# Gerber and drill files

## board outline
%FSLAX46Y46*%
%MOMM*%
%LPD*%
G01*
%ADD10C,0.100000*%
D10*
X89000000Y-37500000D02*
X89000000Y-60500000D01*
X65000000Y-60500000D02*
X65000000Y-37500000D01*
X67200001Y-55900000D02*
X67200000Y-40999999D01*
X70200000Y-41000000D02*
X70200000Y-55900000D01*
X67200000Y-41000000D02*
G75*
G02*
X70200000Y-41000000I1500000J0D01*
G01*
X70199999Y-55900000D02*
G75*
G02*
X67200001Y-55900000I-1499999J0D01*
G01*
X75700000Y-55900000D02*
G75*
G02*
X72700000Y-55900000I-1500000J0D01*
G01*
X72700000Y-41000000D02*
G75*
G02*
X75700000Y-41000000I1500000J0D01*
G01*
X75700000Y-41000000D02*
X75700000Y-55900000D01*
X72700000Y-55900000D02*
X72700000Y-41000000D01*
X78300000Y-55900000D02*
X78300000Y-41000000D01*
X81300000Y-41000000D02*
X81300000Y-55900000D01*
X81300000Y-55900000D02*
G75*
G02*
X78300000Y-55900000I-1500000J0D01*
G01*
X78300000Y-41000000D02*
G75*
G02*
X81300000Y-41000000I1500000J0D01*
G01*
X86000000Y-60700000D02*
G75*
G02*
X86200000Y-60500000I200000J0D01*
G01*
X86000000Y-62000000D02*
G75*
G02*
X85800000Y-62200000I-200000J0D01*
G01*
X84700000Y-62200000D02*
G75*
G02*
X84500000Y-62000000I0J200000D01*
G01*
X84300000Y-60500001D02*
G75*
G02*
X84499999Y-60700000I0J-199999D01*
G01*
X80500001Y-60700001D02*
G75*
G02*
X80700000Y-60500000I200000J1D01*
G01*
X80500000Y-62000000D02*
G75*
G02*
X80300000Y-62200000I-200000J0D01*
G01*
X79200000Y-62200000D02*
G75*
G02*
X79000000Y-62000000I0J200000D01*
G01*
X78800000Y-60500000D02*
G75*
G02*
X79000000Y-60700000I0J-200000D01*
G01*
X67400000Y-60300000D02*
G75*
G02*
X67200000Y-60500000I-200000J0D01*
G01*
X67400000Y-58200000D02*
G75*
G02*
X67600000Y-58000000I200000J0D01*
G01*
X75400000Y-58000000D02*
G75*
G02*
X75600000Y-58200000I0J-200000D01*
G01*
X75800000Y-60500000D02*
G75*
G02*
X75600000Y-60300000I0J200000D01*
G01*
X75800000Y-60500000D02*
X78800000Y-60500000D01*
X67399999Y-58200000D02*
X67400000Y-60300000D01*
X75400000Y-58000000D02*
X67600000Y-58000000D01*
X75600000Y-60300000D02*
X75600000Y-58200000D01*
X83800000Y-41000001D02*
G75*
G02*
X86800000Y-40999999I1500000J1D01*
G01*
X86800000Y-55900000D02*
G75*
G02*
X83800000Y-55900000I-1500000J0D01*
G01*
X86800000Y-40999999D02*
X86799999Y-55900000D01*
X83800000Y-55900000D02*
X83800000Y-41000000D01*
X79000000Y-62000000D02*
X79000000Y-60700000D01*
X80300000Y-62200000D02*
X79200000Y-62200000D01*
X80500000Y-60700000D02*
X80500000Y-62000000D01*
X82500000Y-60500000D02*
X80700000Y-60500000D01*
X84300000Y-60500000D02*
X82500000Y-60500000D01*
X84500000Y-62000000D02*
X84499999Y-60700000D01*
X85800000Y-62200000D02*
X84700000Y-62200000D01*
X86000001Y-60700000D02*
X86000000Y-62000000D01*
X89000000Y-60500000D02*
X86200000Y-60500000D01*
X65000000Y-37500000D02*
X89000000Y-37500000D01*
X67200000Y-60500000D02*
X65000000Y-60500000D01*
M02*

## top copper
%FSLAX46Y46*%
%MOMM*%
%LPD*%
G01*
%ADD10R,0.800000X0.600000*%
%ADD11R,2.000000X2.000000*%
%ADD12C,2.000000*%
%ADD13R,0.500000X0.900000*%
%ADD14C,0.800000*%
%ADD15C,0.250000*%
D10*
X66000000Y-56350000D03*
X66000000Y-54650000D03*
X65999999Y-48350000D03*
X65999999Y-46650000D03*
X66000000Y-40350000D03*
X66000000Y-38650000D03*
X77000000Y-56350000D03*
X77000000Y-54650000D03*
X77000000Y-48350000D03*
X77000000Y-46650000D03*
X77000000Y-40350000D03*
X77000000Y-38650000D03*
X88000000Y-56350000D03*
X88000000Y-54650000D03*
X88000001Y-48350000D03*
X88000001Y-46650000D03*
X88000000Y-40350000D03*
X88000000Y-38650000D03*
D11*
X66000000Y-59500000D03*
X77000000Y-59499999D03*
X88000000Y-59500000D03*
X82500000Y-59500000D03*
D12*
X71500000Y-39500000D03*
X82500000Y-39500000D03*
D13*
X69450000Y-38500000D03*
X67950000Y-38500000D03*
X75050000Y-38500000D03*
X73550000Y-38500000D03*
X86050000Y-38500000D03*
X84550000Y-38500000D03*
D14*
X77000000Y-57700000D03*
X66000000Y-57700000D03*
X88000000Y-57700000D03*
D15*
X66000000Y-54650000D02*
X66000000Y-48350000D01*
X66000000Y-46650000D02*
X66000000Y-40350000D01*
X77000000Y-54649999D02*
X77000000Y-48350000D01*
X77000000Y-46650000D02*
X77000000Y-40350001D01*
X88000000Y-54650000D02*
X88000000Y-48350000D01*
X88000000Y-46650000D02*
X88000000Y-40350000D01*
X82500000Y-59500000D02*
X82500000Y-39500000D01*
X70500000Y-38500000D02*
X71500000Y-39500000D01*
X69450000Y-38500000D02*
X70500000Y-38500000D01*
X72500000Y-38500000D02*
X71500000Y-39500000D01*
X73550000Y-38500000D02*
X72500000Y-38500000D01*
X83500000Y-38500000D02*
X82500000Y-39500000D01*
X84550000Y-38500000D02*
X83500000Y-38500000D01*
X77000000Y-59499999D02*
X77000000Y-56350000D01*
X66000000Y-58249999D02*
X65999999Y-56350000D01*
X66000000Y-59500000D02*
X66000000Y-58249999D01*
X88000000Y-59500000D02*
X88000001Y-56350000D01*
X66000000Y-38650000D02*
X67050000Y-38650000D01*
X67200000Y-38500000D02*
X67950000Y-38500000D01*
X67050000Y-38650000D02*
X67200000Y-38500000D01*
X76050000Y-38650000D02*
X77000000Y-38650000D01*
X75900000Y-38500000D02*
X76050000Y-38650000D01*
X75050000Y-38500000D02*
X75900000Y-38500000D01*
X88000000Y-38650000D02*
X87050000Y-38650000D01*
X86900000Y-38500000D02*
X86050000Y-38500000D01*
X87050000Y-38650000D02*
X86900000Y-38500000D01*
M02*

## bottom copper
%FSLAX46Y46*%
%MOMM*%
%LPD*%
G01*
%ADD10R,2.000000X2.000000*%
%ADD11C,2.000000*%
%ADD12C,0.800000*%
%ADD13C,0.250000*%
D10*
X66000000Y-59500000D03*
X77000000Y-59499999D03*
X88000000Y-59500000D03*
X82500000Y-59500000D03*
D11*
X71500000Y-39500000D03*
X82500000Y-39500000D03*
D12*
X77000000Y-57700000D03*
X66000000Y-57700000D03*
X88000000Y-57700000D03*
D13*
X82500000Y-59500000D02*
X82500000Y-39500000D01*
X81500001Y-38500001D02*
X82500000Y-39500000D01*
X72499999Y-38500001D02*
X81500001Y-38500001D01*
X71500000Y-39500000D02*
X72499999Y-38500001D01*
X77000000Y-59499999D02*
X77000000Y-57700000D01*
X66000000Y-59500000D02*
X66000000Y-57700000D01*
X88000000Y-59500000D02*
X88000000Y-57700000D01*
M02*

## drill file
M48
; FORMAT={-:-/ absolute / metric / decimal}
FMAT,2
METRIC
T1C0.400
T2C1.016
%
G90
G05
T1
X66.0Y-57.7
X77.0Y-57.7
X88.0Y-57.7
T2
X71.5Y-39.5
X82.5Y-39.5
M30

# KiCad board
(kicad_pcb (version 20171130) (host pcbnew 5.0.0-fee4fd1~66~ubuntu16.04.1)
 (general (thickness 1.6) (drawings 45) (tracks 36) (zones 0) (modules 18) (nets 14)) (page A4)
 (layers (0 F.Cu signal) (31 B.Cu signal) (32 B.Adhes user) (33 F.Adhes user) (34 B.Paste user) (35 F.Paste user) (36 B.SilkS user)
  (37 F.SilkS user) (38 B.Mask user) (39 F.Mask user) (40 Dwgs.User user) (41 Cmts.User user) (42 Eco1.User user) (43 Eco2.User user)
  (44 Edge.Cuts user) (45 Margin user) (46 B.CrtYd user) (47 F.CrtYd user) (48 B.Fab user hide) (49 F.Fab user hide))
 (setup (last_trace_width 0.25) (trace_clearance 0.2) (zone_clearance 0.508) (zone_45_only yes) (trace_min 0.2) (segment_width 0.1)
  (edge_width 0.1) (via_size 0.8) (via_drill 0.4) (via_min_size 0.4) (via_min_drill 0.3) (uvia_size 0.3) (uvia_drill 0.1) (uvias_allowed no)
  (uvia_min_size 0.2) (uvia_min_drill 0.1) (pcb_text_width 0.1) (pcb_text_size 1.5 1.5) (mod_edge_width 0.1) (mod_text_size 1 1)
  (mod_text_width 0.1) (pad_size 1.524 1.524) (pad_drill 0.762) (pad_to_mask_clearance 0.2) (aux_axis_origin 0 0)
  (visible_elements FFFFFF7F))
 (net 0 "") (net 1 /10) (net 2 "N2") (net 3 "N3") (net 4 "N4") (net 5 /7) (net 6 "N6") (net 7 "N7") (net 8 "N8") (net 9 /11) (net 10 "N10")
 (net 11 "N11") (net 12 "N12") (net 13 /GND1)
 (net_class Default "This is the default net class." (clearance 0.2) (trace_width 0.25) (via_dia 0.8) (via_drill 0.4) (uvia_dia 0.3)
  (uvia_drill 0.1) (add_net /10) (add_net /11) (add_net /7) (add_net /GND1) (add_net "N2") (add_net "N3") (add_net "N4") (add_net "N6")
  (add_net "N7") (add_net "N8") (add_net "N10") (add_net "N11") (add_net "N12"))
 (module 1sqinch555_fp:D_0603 (layer F.Cu) (at 66 55.5 270)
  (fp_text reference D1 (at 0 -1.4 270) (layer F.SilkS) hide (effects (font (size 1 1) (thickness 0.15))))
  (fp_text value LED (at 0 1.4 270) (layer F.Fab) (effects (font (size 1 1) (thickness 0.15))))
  (pad 2 smd rect (at 0.85 0 270) (size 0.6 0.8) (layers F.Cu F.Paste F.Mask) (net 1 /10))
  (pad 1 smd rect (at -0.85 0 270) (size 0.6 0.8) (layers F.Cu F.Paste F.Mask) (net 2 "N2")))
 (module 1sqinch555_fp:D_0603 (layer F.Cu) (at 65.999999 47.5 270)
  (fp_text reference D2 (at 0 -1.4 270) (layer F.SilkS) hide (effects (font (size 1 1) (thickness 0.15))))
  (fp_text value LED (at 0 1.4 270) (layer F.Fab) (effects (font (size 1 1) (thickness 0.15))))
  (pad 2 smd rect (at 0.85 0 270) (size 0.6 0.8) (layers F.Cu F.Paste F.Mask) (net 2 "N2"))
  (pad 1 smd rect (at -0.85 0 270) (size 0.6 0.8) (layers F.Cu F.Paste F.Mask) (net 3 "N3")))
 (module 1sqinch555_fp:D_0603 (layer F.Cu) (at 66 39.5 270)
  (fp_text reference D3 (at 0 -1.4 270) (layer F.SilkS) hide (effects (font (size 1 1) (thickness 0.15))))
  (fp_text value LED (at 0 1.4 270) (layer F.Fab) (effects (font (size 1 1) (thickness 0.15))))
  (pad 2 smd rect (at 0.85 0 270) (size 0.6 0.8) (layers F.Cu F.Paste F.Mask) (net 3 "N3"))
  (pad 1 smd rect (at -0.85 0 270) (size 0.6 0.8) (layers F.Cu F.Paste F.Mask) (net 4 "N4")))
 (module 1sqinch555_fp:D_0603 (layer F.Cu) (at 77 55.5 270)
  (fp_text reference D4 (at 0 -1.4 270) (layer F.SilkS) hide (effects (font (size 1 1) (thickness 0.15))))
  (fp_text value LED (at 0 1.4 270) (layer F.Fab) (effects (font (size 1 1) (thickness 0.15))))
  (pad 2 smd rect (at 0.85 0 270) (size 0.6 0.8) (layers F.Cu F.Paste F.Mask) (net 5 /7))
  (pad 1 smd rect (at -0.85 0 270) (size 0.6 0.8) (layers F.Cu F.Paste F.Mask) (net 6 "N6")))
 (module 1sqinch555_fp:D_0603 (layer F.Cu) (at 77 47.5 270)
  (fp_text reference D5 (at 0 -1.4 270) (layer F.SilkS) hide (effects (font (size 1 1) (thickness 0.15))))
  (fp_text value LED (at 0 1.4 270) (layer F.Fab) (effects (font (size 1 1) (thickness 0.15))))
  (pad 2 smd rect (at 0.85 0 270) (size 0.6 0.8) (layers F.Cu F.Paste F.Mask) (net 6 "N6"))
  (pad 1 smd rect (at -0.85 0 270) (size 0.6 0.8) (layers F.Cu F.Paste F.Mask) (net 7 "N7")))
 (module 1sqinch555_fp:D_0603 (layer F.Cu) (at 77 39.5 270)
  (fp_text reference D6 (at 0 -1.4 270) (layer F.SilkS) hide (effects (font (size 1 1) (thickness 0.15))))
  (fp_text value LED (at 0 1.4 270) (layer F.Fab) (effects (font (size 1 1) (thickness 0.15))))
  (pad 2 smd rect (at 0.85 0 270) (size 0.6 0.8) (layers F.Cu F.Paste F.Mask) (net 7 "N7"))
  (pad 1 smd rect (at -0.85 0 270) (size 0.6 0.8) (layers F.Cu F.Paste F.Mask) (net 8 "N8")))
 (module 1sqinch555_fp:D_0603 (layer F.Cu) (at 88 55.5 270)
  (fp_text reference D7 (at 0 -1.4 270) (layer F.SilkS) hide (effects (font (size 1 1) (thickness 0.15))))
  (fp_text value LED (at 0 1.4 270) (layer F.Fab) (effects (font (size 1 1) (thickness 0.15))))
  (pad 2 smd rect (at 0.85 0 270) (size 0.6 0.8) (layers F.Cu F.Paste F.Mask) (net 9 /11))
  (pad 1 smd rect (at -0.85 0 270) (size 0.6 0.8) (layers F.Cu F.Paste F.Mask) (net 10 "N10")))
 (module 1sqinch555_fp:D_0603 (layer F.Cu) (at 88.000001 47.5 270)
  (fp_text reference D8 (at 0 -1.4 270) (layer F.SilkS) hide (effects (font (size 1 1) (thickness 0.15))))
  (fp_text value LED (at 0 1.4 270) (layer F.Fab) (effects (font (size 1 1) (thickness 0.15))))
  (pad 2 smd rect (at 0.85 0 270) (size 0.6 0.8) (layers F.Cu F.Paste F.Mask) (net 10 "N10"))
  (pad 1 smd rect (at -0.85 0 270) (size 0.6 0.8) (layers F.Cu F.Paste F.Mask) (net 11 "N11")))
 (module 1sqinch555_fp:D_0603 (layer F.Cu) (at 88 39.5 270)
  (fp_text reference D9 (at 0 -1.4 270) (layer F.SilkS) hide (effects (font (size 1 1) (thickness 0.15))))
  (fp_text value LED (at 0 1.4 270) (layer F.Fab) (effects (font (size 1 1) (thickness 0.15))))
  (pad 2 smd rect (at 0.85 0 270) (size 0.6 0.8) (layers F.Cu F.Paste F.Mask) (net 11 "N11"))
  (pad 1 smd rect (at -0.85 0 270) (size 0.6 0.8) (layers F.Cu F.Paste F.Mask) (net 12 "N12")))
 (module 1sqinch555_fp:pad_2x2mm (layer F.Cu) (at 66 59.5 90)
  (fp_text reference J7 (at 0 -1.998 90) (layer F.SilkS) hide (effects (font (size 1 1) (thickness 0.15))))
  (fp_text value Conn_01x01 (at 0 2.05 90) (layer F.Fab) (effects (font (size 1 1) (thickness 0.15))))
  (pad 1 smd rect (at 0 0 90) (size 2 2) (layers B.Cu B.Mask) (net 1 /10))
  (pad 1 smd rect (at 0 0 90) (size 2 2) (layers F.Cu F.Mask) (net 1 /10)))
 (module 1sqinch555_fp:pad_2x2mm (layer F.Cu) (at 77 59.499999 90)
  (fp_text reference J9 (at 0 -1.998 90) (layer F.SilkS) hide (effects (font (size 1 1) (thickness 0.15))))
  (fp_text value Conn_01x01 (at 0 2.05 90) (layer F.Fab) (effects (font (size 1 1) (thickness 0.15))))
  (pad 1 smd rect (at 0 0 90) (size 2 2) (layers B.Cu B.Mask) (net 5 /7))
  (pad 1 smd rect (at 0 0 90) (size 2 2) (layers F.Cu F.Mask) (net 5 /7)))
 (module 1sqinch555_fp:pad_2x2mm (layer F.Cu) (at 88 59.5 90)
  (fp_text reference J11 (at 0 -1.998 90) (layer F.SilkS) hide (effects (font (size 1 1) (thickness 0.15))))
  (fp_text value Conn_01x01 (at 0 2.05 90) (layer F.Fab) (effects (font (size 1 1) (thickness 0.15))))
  (pad 1 smd rect (at 0 0 90) (size 2 2) (layers B.Cu B.Mask) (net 9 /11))
  (pad 1 smd rect (at 0 0 90) (size 2 2) (layers F.Cu F.Mask) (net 9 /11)))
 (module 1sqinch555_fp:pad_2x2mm (layer F.Cu) (at 82.5 59.5 90)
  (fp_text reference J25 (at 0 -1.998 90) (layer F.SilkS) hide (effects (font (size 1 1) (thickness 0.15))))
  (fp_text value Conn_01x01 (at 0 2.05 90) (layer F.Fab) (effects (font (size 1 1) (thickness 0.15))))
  (pad 1 smd rect (at 0 0 90) (size 2 2) (layers B.Cu B.Mask) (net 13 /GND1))
  (pad 1 smd rect (at 0 0 90) (size 2 2) (layers F.Cu F.Mask) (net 13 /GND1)))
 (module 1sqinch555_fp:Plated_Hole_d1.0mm (layer F.Cu) (at 71.5 39.5 90)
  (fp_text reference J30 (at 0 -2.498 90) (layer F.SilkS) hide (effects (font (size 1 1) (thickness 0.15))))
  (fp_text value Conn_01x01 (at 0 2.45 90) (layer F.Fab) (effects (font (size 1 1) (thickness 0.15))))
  (pad 1 thru_hole circle (at 0 0 90) (size 2 2) (drill 1.016) (layers *.Cu *.Mask) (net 13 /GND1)))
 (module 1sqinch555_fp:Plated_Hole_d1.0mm (layer F.Cu) (at 82.5 39.5 90)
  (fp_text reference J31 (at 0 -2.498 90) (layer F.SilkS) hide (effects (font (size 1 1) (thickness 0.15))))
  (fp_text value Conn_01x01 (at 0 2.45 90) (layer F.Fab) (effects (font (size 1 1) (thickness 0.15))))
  (pad 1 thru_hole circle (at 0 0 90) (size 2 2) (drill 1.016) (layers *.Cu *.Mask) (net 13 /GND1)))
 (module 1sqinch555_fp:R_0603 (layer F.Cu) (at 68.7 38.5 180)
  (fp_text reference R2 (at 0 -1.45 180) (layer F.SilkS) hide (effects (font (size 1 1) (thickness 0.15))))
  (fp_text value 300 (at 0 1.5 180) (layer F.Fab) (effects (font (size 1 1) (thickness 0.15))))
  (pad 1 smd rect (at -0.75 0 180) (size 0.5 0.9) (layers F.Cu F.Paste F.Mask) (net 13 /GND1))
  (pad 2 smd rect (at 0.75 0 180) (size 0.5 0.9) (layers F.Cu F.Paste F.Mask) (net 4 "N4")))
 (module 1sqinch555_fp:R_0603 (layer F.Cu) (at 74.3 38.5)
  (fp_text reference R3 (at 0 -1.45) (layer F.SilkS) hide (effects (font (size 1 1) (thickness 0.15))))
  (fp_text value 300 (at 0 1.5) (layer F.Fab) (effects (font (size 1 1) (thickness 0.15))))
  (pad 2 smd rect (at 0.75 0) (size 0.5 0.9) (layers F.Cu F.Paste F.Mask) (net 8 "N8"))
  (pad 1 smd rect (at -0.75 0) (size 0.5 0.9) (layers F.Cu F.Paste F.Mask) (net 13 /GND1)))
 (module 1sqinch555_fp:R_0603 (layer F.Cu) (at 85.3 38.5)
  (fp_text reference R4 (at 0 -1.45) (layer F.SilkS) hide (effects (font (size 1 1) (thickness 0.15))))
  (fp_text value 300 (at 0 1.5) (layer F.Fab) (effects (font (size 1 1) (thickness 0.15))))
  (pad 2 smd rect (at 0.75 0) (size 0.5 0.9) (layers F.Cu F.Paste F.Mask) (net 12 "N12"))
  (pad 1 smd rect (at -0.75 0) (size 0.5 0.9) (layers F.Cu F.Paste F.Mask) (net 13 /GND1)))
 (gr_line (start 89 37.5) (end 89 60.5) (layer Edge.Cuts) (width 0.1))
 (gr_line (start 65 60.5) (end 65 37.5) (layer Edge.Cuts) (width 0.1))
 (gr_line (start 67.200001 55.9) (end 67.2 40.999999) (layer Edge.Cuts) (width 0.1))
 (gr_line (start 70.2 41) (end 70.2 55.9) (layer Edge.Cuts) (width 0.1))
 (gr_arc (start 68.7 41) (end 70.2 41) (angle -180) (layer Edge.Cuts) (width 0.1))
 (gr_arc (start 68.7 55.9) (end 67.200001 55.9) (angle -180) (layer Edge.Cuts) (width 0.1))
 (gr_arc (start 74.2 55.9) (end 72.7 55.9) (angle -180) (layer Edge.Cuts) (width 0.1))
 (gr_arc (start 74.2 41) (end 75.7 41) (angle -180) (layer Edge.Cuts) (width 0.1))
 (gr_line (start 75.7 41) (end 75.7 55.9) (layer Edge.Cuts) (width 0.1))
 (gr_line (start 72.7 55.9) (end 72.7 41) (layer Edge.Cuts) (width 0.1))
 (gr_line (start 78.3 55.9) (end 78.3 41) (layer Edge.Cuts) (width 0.1))
 (gr_line (start 81.3 41) (end 81.3 55.9) (layer Edge.Cuts) (width 0.1))
 (gr_arc (start 79.8 55.9) (end 78.3 55.9) (angle -180) (layer Edge.Cuts) (width 0.1))
 (gr_arc (start 79.8 41) (end 81.3 41) (angle -180) (layer Edge.Cuts) (width 0.1))
 (gr_arc (start 86.2 60.7) (end 86.2 60.5) (angle -90) (layer Edge.Cuts) (width 0.1))
 (gr_arc (start 85.8 62) (end 85.8 62.2) (angle -90) (layer Edge.Cuts) (width 0.1))
 (gr_arc (start 84.7 62) (end 84.5 62) (angle -90) (layer Edge.Cuts) (width 0.1))
 (gr_arc (start 84.3 60.7) (end 84.499999 60.7) (angle -90) (layer Edge.Cuts) (width 0.1))
 (gr_arc (start 80.700001 60.7) (end 80.7 60.5) (angle -90) (layer Edge.Cuts) (width 0.1))
 (gr_arc (start 80.3 62) (end 80.3 62.2) (angle -90) (layer Edge.Cuts) (width 0.1))
 (gr_arc (start 79.2 62) (end 79 62) (angle -90) (layer Edge.Cuts) (width 0.1))
 (gr_arc (start 78.8 60.7) (end 79 60.7) (angle -90) (layer Edge.Cuts) (width 0.1))
 (gr_arc (start 67.2 60.3) (end 67.2 60.5) (angle -90) (layer Edge.Cuts) (width 0.1))
 (gr_arc (start 67.6 58.2) (end 67.6 58) (angle -90) (layer Edge.Cuts) (width 0.1))
 (gr_arc (start 75.4 58.2) (end 75.6 58.2) (angle -90) (layer Edge.Cuts) (width 0.1))
 (gr_arc (start 75.8 60.3) (end 75.6 60.3) (angle -90) (layer Edge.Cuts) (width 0.1))
 (gr_line (start 75.8 60.5) (end 78.8 60.5) (layer Edge.Cuts) (width 0.1))
 (gr_line (start 67.399999 58.2) (end 67.4 60.3) (layer Edge.Cuts) (width 0.1))
 (gr_line (start 75.4 58) (end 67.6 58) (layer Edge.Cuts) (width 0.1))
 (gr_line (start 75.6 60.3) (end 75.6 58.2) (layer Edge.Cuts) (width 0.1))
 (gr_arc (start 85.3 41) (end 86.8 40.999999) (angle -180) (layer Edge.Cuts) (width 0.1))
 (gr_arc (start 85.3 55.9) (end 83.8 55.9) (angle -180) (layer Edge.Cuts) (width 0.1))
 (gr_line (start 86.8 40.999999) (end 86.799999 55.9) (layer Edge.Cuts) (width 0.1))
 (gr_line (start 83.8 55.9) (end 83.8 41) (layer Edge.Cuts) (width 0.1))
 (gr_line (start 79 62) (end 79 60.7) (layer Edge.Cuts) (width 0.1))
 (gr_line (start 80.3 62.2) (end 79.2 62.2) (layer Edge.Cuts) (width 0.1))
 (gr_line (start 80.5 60.7) (end 80.5 62) (layer Edge.Cuts) (width 0.1))
 (gr_line (start 82.5 60.5) (end 80.7 60.5) (layer Edge.Cuts) (width 0.1))
 (gr_line (start 84.3 60.5) (end 82.5 60.5) (layer Edge.Cuts) (width 0.1))
 (gr_line (start 84.5 62) (end 84.499999 60.7) (layer Edge.Cuts) (width 0.1))
 (gr_line (start 85.8 62.2) (end 84.7 62.2) (layer Edge.Cuts) (width 0.1))
 (gr_line (start 86.000001 60.7) (end 86 62) (layer Edge.Cuts) (width 0.1))
 (gr_line (start 89 60.5) (end 86.2 60.5) (layer Edge.Cuts) (width 0.1))
 (gr_line (start 65 37.5) (end 89 37.5) (layer Edge.Cuts) (width 0.1))
 (gr_line (start 67.2 60.5) (end 65 60.5) (layer Edge.Cuts) (width 0.1))
 (segment (start 66 54.65) (end 66 48.35) (width 0.25) (layer F.Cu) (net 2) (status 30))
 (segment (start 66 46.65) (end 66 40.35) (width 0.25) (layer F.Cu) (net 3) (status 30))
 (segment (start 77 54.649999) (end 77 48.35) (width 0.25) (layer F.Cu) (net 6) (status 30))
 (segment (start 77 46.65) (end 77 40.350001) (width 0.25) (layer F.Cu) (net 7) (status 30))
 (segment (start 88 54.65) (end 88 48.35) (width 0.25) (layer F.Cu) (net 10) (status 30))
 (segment (start 88 46.65) (end 88 40.35) (width 0.25) (layer F.Cu) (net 11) (status 30))
 (segment (start 82.5 59.5) (end 82.5 39.5) (width 0.25) (layer F.Cu) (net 13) (status 30))
 (segment (start 82.5 59.5) (end 82.5 39.5) (width 0.25) (layer B.Cu) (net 13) (status 30))
 (segment (start 70.5 38.5) (end 71.5 39.5) (width 0.25) (layer F.Cu) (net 13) (status 20))
 (segment (start 69.45 38.5) (end 70.5 38.5) (width 0.25) (layer F.Cu) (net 13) (status 10))
 (segment (start 72.5 38.5) (end 71.5 39.5) (width 0.25) (layer F.Cu) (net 13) (status 20))
 (segment (start 73.55 38.5) (end 72.5 38.5) (width 0.25) (layer F.Cu) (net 13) (status 10))
 (segment (start 83.5 38.5) (end 82.5 39.5) (width 0.25) (layer F.Cu) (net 13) (status 20))
 (segment (start 84.55 38.5) (end 83.5 38.5) (width 0.25) (layer F.Cu) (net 13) (status 10))
 (segment (start 81.500001 38.500001) (end 82.5 39.5) (width 0.25) (layer B.Cu) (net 13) (status 20))
 (segment (start 72.499999 38.500001) (end 81.500001 38.500001) (width 0.25) (layer B.Cu) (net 13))
 (segment (start 71.5 39.5) (end 72.499999 38.500001) (width 0.25) (layer B.Cu) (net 13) (status 10))
 (segment (start 77 59.499999) (end 77 56.35) (width 0.25) (layer F.Cu) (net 5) (status 30))
 (via (at 77 57.7) (size 0.8) (drill 0.4) (layers F.Cu B.Cu) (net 5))
 (segment (start 77 59.499999) (end 77 57.7) (width 0.25) (layer B.Cu) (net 5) (status 10))
 (segment (start 66 58.249999) (end 65.999999 56.35) (width 0.25) (layer F.Cu) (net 1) (status 20))
 (segment (start 66 59.5) (end 66 58.249999) (width 0.25) (layer F.Cu) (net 1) (status 10))
 (via (at 66 57.7) (size 0.8) (drill 0.4) (layers F.Cu B.Cu) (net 1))
 (segment (start 66 59.5) (end 66 57.7) (width 0.25) (layer B.Cu) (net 1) (status 10))
 (segment (start 88 59.5) (end 88.000001 56.35) (width 0.25) (layer F.Cu) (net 9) (status 30))
 (via (at 88 57.7) (size 0.8) (drill 0.4) (layers F.Cu B.Cu) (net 9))
 (segment (start 88 59.5) (end 88 57.7) (width 0.25) (layer B.Cu) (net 9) (status 10))
 (segment (start 66 38.65) (end 67.05 38.65) (width 0.25) (layer F.Cu) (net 4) (status 10))
 (segment (start 67.2 38.5) (end 67.95 38.5) (width 0.25) (layer F.Cu) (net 4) (status 20))
 (segment (start 67.05 38.65) (end 67.2 38.5) (width 0.25) (layer F.Cu) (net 4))
 (segment (start 76.05 38.65) (end 77 38.65) (width 0.25) (layer F.Cu) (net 8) (status 20))
 (segment (start 75.9 38.5) (end 76.05 38.65) (width 0.25) (layer F.Cu) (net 8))
 (segment (start 75.05 38.5) (end 75.9 38.5) (width 0.25) (layer F.Cu) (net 8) (status 10))
 (segment (start 88 38.65) (end 87.05 38.65) (width 0.25) (layer F.Cu) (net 12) (status 10))
 (segment (start 86.9 38.5) (end 86.05 38.5) (width 0.25) (layer F.Cu) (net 12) (status 20))
 (segment (start 87.05 38.65) (end 86.9 38.5) (width 0.25) (layer F.Cu) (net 12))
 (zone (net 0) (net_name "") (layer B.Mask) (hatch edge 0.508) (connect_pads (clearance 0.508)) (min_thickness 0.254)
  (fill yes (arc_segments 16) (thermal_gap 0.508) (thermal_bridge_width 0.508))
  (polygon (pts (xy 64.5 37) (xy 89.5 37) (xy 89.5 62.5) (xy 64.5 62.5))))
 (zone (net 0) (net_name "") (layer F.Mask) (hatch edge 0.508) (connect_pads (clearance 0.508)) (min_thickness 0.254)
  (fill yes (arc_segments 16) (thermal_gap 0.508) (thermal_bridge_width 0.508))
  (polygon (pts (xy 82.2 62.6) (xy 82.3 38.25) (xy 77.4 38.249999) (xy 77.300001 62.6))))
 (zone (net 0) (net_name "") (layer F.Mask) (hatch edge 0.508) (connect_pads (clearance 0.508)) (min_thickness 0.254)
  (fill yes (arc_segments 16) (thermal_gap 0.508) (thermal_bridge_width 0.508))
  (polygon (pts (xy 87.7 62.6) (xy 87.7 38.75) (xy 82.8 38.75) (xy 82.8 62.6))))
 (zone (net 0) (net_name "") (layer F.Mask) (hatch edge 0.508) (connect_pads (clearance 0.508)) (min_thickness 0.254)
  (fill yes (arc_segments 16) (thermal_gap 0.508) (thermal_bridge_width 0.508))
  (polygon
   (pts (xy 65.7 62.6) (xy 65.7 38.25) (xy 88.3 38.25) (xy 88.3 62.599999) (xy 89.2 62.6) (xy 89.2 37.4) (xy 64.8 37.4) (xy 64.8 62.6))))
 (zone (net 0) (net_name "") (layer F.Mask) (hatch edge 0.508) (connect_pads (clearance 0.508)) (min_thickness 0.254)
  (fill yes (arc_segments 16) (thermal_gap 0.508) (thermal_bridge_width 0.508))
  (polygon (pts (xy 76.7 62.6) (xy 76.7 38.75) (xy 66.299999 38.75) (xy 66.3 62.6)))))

